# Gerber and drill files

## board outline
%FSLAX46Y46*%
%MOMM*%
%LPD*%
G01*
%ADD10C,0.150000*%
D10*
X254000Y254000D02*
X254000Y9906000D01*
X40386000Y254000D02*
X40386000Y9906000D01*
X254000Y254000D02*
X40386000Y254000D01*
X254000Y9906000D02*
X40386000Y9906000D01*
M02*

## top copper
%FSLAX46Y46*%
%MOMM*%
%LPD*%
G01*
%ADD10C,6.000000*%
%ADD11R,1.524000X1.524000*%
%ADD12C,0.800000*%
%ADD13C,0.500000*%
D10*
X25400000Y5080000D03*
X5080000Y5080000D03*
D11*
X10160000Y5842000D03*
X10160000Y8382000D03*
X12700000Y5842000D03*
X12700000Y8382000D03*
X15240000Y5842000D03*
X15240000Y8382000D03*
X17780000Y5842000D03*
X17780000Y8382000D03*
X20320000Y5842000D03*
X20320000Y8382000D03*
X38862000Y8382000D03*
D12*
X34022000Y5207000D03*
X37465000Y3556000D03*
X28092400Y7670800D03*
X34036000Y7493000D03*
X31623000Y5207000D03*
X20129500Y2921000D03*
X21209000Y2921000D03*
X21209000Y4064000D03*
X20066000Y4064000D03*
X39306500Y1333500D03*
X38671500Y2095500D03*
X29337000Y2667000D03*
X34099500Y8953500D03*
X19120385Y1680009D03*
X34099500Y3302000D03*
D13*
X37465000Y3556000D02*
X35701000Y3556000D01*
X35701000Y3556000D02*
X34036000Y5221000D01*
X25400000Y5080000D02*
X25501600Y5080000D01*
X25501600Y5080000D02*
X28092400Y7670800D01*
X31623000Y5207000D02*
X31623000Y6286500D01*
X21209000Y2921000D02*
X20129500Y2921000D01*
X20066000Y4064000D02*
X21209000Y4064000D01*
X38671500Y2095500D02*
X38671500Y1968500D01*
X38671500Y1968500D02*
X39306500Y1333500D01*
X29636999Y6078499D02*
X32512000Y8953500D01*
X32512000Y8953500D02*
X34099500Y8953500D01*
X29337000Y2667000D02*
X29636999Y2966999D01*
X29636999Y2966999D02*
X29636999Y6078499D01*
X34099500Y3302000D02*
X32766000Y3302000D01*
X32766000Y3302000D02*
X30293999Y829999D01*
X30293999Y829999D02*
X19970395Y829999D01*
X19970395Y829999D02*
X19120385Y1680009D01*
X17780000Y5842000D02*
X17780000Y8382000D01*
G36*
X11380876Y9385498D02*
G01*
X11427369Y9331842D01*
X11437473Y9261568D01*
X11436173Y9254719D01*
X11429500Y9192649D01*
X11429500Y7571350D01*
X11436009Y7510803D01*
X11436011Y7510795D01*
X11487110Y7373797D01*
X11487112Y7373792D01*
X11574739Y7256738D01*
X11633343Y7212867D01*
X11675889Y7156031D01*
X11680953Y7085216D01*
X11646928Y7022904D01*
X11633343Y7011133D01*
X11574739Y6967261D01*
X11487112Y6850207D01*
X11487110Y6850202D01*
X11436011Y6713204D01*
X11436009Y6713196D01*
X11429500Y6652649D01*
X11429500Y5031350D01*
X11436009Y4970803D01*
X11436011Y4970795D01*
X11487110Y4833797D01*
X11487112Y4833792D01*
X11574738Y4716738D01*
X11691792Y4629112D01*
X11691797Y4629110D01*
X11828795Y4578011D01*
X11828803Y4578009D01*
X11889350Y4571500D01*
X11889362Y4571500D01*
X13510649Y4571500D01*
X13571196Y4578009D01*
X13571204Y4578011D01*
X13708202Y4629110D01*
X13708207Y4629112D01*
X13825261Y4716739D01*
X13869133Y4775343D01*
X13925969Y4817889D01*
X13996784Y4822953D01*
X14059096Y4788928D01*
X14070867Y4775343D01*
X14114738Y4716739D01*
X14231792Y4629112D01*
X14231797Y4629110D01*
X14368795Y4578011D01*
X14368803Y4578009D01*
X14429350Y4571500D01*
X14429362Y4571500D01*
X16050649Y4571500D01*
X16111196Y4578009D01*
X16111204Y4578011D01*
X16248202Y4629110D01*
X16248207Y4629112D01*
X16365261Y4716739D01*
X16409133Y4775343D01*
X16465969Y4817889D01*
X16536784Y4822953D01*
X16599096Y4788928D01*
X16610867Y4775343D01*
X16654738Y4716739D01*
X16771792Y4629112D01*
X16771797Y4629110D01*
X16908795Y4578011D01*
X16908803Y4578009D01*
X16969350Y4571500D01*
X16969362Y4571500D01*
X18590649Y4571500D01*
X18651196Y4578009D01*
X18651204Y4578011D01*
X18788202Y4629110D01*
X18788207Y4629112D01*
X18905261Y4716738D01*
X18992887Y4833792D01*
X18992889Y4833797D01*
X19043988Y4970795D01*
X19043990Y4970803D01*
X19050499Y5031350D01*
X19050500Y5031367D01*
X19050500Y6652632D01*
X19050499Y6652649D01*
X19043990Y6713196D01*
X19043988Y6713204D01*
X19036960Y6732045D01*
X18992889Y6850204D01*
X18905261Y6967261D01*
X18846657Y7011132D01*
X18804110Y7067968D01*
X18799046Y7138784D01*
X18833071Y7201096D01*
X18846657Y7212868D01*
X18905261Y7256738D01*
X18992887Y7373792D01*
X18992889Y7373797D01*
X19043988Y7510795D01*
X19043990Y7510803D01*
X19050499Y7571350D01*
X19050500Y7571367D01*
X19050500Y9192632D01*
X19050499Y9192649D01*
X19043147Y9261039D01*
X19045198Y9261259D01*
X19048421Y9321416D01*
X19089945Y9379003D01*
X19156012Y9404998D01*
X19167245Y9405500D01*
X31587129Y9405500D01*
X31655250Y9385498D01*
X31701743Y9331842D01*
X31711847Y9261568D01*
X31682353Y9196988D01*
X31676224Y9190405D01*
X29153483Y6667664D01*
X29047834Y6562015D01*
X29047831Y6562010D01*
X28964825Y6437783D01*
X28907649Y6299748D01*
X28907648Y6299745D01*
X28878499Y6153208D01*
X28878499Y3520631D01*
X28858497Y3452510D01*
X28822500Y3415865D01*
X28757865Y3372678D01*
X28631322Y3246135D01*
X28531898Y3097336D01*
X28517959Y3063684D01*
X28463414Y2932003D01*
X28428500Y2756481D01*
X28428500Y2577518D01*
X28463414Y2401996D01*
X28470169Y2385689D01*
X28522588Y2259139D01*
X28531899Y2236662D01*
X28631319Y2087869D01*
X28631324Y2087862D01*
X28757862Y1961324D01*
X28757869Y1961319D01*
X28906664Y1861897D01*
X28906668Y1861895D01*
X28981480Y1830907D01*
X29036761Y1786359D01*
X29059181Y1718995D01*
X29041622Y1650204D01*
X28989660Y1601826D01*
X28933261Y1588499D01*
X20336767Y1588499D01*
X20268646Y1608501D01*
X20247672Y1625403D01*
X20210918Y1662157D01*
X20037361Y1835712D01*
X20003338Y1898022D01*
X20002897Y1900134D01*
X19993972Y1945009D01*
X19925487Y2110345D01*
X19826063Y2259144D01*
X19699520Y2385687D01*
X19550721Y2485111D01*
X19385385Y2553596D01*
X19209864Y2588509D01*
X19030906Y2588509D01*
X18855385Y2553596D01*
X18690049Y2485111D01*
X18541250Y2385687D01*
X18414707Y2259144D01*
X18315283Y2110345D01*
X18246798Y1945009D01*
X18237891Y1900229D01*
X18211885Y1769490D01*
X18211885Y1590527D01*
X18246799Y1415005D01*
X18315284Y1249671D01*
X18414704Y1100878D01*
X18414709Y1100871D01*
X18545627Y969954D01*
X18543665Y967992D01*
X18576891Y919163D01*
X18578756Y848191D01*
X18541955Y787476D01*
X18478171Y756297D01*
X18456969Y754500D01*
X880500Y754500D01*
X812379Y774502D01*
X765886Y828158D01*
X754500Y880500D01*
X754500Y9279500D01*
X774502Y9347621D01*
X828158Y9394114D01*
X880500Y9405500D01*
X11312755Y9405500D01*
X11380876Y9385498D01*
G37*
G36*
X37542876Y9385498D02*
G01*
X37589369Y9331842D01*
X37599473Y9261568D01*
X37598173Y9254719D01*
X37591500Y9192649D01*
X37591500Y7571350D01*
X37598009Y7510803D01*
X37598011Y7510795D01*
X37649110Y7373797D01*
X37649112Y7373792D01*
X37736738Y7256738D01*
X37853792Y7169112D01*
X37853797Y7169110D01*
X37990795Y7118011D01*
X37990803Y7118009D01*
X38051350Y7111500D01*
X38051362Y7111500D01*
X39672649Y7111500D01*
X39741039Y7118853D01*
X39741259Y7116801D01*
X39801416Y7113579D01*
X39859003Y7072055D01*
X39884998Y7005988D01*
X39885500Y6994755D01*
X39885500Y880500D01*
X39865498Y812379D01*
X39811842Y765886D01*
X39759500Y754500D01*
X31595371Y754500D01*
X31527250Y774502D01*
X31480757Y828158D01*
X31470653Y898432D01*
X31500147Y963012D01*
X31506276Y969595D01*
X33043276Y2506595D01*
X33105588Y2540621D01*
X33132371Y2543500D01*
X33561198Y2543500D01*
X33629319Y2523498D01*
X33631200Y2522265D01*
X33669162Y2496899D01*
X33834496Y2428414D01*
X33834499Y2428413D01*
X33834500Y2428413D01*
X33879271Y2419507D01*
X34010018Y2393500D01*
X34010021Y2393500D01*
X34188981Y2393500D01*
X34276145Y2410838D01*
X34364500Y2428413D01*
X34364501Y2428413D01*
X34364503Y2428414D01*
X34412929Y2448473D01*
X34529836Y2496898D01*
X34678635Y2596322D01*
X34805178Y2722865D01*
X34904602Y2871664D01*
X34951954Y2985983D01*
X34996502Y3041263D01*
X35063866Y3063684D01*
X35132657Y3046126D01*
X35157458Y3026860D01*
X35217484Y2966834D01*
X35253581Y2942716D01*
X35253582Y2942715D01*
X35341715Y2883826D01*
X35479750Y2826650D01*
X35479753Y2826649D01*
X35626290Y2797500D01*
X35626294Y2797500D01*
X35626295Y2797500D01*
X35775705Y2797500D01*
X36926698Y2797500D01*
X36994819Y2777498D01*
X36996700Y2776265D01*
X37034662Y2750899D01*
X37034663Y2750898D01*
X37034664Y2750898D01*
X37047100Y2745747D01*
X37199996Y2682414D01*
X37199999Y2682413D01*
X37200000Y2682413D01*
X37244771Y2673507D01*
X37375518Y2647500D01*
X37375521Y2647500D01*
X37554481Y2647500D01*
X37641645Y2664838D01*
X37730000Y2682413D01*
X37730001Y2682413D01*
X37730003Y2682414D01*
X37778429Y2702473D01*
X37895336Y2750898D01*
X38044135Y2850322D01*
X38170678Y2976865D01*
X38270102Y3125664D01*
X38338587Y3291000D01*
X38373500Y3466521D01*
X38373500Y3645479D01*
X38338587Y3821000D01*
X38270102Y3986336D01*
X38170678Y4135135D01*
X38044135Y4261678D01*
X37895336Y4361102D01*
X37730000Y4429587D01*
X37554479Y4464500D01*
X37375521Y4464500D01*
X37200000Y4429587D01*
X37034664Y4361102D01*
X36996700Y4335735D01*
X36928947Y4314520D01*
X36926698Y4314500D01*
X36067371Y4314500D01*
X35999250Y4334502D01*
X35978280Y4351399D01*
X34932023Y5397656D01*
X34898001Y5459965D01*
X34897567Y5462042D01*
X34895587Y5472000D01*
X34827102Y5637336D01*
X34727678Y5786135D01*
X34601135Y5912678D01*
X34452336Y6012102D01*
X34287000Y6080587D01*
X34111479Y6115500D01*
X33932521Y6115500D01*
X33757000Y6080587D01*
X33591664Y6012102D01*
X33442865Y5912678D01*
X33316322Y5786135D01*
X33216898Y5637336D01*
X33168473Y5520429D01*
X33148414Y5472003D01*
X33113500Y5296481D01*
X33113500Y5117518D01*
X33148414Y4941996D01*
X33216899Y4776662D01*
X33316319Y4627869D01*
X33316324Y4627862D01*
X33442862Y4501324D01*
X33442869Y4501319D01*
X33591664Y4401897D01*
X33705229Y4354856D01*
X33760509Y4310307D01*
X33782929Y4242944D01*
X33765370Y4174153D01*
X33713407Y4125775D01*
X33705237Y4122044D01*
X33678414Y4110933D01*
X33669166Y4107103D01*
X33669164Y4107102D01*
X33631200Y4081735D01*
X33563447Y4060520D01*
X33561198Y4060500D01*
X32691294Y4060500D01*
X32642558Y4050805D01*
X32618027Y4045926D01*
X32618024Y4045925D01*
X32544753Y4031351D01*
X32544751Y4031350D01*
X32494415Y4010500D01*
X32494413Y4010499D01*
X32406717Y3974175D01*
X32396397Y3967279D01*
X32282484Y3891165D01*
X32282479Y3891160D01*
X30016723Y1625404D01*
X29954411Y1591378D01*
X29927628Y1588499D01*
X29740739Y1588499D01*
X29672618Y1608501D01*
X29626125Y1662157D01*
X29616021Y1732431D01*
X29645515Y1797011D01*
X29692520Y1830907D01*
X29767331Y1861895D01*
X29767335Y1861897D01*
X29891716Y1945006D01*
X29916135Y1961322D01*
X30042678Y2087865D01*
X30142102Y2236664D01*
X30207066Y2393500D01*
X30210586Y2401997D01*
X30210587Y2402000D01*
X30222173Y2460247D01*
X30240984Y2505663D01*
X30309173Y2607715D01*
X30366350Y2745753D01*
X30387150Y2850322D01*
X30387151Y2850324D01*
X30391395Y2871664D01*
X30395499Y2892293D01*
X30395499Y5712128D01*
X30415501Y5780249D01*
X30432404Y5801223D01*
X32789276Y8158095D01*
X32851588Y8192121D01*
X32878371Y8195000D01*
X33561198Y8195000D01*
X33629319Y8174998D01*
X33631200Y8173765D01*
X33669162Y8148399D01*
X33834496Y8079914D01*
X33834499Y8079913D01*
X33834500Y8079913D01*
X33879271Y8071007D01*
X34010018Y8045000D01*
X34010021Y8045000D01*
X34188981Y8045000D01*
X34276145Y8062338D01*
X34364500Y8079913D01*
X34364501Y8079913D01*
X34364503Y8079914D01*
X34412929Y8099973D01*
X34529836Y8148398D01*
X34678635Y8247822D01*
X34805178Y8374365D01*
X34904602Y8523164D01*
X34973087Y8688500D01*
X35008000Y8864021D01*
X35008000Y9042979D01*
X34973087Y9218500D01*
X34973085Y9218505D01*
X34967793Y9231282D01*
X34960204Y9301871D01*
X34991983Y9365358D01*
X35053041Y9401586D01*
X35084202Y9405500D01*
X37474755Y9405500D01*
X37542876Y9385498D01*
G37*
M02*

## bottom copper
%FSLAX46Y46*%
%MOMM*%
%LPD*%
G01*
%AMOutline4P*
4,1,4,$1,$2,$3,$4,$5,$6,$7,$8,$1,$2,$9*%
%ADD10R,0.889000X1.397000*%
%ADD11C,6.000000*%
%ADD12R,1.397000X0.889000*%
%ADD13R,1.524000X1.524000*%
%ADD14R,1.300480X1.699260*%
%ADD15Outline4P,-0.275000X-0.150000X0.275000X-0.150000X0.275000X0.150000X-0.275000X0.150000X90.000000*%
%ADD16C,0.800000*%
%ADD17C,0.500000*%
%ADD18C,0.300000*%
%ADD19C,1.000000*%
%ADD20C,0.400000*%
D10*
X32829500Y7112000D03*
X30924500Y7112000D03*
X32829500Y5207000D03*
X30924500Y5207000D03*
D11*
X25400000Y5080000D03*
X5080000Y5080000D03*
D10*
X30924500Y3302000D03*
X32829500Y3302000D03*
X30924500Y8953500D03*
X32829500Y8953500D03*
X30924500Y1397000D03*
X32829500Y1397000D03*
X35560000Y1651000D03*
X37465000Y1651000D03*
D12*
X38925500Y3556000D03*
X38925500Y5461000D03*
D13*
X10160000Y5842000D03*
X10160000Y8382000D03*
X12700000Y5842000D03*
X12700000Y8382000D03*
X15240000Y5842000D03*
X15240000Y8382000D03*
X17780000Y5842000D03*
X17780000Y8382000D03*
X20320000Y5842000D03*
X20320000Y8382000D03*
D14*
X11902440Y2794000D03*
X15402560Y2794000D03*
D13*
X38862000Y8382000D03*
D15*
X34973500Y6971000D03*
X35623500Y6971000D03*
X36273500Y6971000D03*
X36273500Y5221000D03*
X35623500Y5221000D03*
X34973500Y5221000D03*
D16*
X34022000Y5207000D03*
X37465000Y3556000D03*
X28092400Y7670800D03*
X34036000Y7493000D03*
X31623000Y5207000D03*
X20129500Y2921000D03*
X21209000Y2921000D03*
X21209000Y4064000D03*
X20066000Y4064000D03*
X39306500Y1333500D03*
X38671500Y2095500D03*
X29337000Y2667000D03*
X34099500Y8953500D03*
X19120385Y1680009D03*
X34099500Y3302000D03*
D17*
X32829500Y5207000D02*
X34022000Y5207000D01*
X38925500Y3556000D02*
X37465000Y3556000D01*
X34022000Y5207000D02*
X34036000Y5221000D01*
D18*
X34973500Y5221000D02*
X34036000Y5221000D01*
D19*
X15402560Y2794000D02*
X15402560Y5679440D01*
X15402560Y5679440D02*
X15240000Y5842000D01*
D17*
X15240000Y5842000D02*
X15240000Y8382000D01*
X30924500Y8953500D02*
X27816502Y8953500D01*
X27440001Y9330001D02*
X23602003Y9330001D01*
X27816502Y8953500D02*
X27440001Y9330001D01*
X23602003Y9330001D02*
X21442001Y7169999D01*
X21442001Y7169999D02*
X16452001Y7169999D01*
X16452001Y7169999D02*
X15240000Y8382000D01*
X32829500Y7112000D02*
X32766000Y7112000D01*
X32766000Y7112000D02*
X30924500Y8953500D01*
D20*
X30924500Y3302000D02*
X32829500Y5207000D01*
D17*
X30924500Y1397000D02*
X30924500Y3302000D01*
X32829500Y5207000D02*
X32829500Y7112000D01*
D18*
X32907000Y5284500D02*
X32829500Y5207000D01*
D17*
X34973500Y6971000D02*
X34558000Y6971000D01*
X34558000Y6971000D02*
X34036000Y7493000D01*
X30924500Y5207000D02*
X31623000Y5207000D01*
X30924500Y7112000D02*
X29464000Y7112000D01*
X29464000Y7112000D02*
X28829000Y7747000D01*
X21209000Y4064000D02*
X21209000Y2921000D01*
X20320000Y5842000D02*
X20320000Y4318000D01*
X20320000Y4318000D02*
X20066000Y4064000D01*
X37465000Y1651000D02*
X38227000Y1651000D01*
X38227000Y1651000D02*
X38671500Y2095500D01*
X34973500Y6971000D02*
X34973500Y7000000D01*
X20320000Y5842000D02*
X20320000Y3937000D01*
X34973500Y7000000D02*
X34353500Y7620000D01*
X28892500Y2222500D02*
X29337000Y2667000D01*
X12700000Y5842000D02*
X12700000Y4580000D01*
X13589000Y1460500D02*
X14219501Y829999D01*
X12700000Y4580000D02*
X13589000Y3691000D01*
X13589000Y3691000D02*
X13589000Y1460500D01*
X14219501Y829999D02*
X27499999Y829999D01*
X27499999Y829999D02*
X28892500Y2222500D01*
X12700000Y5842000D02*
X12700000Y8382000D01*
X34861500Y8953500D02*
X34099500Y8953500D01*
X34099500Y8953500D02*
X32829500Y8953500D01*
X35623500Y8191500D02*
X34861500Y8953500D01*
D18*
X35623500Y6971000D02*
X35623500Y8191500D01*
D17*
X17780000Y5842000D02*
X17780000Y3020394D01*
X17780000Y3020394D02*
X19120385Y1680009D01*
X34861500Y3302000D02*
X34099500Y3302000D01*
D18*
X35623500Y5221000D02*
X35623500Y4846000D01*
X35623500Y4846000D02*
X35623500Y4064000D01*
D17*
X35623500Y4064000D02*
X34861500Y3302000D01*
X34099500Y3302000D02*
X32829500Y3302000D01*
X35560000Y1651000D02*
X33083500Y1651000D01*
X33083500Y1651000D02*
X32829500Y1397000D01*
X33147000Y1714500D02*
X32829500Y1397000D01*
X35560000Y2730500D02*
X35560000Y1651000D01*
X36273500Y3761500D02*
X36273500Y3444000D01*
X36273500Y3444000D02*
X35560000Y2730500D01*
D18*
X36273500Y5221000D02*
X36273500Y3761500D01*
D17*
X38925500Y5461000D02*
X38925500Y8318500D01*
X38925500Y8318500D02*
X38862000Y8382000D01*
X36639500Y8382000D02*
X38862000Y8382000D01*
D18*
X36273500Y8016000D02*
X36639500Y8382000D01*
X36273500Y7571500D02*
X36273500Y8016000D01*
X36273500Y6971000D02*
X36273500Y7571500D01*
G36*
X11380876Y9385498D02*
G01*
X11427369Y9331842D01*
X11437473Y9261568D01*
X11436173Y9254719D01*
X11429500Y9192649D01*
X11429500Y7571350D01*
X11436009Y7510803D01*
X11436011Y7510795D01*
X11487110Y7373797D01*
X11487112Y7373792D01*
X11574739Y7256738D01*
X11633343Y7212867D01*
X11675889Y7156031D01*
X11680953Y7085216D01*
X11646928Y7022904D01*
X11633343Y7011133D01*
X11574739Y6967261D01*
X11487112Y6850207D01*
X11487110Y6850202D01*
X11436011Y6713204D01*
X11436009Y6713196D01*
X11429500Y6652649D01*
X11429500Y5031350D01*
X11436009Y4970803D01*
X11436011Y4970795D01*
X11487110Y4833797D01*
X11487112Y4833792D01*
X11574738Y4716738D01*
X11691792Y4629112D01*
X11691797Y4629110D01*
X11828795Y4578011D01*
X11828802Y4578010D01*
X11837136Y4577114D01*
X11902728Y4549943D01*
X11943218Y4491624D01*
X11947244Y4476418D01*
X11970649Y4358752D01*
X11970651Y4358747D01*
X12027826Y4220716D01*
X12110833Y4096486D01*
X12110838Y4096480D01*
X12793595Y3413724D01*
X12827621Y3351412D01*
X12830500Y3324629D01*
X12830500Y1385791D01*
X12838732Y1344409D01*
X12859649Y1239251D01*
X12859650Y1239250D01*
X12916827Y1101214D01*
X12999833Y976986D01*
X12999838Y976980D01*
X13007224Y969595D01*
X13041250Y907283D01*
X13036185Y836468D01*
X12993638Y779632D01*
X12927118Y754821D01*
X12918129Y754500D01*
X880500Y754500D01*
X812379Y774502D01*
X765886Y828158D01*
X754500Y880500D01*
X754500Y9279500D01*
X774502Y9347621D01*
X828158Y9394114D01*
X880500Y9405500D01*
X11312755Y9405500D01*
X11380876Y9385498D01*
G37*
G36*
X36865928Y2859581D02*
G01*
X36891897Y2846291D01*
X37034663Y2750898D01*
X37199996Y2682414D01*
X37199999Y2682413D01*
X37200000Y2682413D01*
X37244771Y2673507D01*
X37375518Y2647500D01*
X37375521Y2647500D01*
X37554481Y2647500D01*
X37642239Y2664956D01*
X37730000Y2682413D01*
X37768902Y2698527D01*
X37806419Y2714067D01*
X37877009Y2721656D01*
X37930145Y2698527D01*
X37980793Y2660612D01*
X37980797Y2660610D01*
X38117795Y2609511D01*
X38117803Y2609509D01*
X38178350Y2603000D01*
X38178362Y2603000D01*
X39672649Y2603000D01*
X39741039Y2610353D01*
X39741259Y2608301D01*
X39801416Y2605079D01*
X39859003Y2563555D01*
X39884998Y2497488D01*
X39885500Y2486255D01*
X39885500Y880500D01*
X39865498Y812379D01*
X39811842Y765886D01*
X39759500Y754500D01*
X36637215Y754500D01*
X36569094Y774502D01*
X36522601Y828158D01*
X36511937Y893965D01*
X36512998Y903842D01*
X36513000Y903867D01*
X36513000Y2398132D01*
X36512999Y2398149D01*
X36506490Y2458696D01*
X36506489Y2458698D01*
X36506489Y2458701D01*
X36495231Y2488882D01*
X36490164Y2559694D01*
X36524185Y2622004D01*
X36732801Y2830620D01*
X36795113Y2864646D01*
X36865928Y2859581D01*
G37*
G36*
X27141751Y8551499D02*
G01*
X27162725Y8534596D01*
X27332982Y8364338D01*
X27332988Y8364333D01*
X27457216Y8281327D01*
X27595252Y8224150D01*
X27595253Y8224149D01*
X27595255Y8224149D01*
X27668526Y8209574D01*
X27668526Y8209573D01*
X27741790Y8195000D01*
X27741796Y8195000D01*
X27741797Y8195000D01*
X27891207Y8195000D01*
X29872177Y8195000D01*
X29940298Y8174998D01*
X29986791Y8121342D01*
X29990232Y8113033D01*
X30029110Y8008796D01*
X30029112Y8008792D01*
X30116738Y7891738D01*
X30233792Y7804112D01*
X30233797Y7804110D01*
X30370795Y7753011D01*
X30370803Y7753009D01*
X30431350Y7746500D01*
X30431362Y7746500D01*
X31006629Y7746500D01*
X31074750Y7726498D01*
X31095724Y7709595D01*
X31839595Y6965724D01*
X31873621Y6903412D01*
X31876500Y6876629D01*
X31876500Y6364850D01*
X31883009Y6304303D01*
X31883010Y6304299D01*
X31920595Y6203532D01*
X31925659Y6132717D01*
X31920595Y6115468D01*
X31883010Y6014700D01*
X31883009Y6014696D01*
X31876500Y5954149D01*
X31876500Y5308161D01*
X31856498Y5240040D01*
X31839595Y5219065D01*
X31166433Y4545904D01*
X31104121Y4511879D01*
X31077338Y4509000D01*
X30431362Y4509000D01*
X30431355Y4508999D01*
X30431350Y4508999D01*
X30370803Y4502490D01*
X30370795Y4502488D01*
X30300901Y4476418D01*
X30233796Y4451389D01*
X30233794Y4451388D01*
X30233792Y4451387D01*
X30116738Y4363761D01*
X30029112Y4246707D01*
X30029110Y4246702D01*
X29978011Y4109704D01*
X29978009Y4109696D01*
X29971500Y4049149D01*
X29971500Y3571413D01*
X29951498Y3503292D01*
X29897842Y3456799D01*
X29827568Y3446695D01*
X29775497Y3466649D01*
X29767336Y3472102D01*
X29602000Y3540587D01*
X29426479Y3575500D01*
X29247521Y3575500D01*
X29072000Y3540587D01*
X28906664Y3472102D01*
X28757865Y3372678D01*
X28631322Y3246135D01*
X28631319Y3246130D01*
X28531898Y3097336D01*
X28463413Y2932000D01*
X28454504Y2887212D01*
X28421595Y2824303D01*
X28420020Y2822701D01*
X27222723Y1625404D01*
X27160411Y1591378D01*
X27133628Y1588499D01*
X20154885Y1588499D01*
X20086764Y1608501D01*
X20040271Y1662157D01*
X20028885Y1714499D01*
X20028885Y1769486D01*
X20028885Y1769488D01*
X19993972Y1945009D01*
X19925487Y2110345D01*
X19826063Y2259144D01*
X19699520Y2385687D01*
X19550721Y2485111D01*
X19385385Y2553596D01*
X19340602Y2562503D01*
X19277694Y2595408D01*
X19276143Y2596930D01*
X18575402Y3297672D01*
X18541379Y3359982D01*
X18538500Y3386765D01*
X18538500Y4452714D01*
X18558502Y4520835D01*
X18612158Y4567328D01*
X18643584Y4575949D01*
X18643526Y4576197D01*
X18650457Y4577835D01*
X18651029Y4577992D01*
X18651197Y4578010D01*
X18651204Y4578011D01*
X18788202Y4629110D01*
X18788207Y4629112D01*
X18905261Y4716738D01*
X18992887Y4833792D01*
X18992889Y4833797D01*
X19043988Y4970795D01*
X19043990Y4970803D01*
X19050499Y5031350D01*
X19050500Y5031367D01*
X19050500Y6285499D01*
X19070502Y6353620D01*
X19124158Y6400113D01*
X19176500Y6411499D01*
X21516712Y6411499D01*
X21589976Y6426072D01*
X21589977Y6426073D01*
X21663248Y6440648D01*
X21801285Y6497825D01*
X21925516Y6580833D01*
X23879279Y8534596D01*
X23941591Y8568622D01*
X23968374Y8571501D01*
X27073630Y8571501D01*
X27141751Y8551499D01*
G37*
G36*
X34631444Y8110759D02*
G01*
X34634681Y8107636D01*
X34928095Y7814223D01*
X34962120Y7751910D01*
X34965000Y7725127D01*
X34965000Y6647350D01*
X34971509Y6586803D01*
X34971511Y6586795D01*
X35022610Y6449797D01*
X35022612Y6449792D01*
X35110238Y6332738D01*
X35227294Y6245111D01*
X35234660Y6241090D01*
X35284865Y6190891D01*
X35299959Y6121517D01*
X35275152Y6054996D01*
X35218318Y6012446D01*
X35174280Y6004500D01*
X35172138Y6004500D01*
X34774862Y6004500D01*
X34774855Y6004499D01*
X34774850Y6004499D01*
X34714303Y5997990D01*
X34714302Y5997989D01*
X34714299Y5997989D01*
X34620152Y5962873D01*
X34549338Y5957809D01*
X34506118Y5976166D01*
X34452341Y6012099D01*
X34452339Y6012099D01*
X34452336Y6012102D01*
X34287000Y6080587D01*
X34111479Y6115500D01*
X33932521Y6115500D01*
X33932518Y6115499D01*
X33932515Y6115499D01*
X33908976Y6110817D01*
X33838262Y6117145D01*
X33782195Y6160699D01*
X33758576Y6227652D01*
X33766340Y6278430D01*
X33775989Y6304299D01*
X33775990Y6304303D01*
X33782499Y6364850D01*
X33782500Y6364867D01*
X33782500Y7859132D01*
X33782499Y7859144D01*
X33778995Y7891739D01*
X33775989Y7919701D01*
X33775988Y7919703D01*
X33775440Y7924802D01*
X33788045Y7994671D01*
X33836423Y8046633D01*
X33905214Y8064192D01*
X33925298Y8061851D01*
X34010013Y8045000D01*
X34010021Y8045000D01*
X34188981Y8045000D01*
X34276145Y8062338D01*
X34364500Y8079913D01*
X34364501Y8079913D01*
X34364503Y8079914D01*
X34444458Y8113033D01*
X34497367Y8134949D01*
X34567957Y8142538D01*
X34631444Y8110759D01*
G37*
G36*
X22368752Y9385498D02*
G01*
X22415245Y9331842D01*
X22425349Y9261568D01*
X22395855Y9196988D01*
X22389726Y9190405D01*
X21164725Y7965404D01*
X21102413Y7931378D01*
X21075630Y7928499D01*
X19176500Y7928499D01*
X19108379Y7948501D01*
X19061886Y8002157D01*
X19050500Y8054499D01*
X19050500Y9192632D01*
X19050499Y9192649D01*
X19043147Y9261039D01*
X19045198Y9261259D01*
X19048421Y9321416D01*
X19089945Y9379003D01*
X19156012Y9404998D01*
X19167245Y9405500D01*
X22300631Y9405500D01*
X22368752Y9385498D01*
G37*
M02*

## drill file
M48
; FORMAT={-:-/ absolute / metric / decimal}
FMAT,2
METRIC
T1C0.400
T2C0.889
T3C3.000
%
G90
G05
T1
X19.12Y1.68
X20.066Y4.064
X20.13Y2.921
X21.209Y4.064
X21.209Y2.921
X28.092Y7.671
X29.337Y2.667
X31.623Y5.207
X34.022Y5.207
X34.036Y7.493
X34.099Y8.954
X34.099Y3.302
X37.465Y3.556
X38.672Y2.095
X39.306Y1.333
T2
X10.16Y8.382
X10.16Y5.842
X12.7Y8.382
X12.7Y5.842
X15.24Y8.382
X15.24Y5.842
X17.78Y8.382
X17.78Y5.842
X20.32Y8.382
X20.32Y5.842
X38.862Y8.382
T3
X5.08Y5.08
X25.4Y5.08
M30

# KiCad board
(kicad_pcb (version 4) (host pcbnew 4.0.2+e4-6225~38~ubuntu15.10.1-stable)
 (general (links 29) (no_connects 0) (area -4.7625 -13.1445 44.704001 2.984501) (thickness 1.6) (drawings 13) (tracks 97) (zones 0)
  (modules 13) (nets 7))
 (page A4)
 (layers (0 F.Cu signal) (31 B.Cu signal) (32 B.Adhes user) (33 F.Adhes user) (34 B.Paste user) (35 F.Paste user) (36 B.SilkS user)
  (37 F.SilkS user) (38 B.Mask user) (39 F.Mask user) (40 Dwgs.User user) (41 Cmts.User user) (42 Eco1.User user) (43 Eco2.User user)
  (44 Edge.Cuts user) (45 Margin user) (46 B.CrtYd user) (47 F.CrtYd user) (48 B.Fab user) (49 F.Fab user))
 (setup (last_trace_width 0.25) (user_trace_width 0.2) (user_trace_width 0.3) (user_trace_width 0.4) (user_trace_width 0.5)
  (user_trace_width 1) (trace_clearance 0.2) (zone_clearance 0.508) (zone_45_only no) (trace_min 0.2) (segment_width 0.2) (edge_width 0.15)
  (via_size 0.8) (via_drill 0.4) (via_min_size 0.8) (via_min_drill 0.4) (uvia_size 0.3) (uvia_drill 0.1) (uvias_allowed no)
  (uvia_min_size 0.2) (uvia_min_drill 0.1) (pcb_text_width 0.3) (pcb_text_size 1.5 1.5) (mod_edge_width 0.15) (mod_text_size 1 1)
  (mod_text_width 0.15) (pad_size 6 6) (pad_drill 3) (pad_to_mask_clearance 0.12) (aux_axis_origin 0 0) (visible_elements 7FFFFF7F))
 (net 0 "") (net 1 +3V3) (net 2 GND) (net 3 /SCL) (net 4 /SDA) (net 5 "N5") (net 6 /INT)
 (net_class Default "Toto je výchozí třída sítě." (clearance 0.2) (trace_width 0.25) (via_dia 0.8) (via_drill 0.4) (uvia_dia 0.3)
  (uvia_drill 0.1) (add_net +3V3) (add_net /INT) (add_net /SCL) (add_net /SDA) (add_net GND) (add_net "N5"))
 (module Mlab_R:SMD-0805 (layer B.Cu) (at 31.877 -7.112 180)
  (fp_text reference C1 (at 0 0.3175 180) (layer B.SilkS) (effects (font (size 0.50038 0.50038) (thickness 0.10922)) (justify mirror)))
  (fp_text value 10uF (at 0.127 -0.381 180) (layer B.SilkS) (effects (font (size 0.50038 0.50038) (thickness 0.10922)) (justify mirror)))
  (pad 1 smd rect (at -0.9525 0 180) (size 0.889 1.397) (layers B.Cu B.Paste B.Mask) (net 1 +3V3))
  (pad 2 smd rect (at 0.9525 0 180) (size 0.889 1.397) (layers B.Cu B.Paste B.Mask) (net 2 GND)))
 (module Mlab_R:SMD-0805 (layer B.Cu) (at 31.877 -5.207 180)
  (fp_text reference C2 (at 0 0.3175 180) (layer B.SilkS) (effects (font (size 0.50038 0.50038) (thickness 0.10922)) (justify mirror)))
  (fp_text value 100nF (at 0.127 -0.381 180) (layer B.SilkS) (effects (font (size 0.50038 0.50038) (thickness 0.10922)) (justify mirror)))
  (pad 1 smd rect (at -0.9525 0 180) (size 0.889 1.397) (layers B.Cu B.Paste B.Mask) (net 1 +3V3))
  (pad 2 smd rect (at 0.9525 0 180) (size 0.889 1.397) (layers B.Cu B.Paste B.Mask) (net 2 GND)))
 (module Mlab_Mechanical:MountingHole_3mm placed (layer F.Cu) (at 25.4 -5.08)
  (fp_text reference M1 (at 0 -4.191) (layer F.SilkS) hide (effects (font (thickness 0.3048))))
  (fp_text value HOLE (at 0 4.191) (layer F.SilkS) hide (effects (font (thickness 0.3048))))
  (pad 1 thru_hole circle (at 0 0) (size 6 6) (drill 3) (layers *.Cu *.Adhes *.Mask) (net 2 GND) (clearance 1) (zone_connect 2)))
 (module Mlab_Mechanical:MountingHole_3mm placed (layer F.Cu) (at 5.08 -5.08)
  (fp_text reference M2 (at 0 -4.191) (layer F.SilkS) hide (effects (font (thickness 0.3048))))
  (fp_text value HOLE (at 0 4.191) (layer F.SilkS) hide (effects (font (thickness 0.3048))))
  (pad 1 thru_hole circle (at 0 0) (size 6 6) (drill 3) (layers *.Cu *.Adhes *.Mask) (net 2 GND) (clearance 1) (zone_connect 2)))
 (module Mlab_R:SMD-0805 (layer B.Cu) (at 31.877 -3.302)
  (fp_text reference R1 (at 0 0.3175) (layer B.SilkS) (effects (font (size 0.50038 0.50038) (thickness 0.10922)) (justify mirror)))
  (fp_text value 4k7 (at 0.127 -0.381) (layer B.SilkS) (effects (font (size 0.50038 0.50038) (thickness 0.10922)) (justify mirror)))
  (pad 1 smd rect (at -0.9525 0) (size 0.889 1.397) (layers B.Cu B.Paste B.Mask) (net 1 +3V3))
  (pad 2 smd rect (at 0.9525 0) (size 0.889 1.397) (layers B.Cu B.Paste B.Mask) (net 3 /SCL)))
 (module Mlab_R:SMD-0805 (layer B.Cu) (at 31.877 -8.9535)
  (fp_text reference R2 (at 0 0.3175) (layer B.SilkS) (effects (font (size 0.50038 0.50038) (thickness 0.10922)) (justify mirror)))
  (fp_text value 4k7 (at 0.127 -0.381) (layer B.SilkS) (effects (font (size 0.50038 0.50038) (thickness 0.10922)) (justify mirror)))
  (pad 1 smd rect (at -0.9525 0) (size 0.889 1.397) (layers B.Cu B.Paste B.Mask) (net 1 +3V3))
  (pad 2 smd rect (at 0.9525 0) (size 0.889 1.397) (layers B.Cu B.Paste B.Mask) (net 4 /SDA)))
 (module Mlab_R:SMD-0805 (layer B.Cu) (at 31.877 -1.397)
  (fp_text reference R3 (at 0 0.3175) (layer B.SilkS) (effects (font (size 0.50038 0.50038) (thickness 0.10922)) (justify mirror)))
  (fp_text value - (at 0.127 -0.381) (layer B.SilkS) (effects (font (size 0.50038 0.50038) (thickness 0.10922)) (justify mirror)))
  (pad 1 smd rect (at -0.9525 0) (size 0.889 1.397) (layers B.Cu B.Paste B.Mask) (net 1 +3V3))
  (pad 2 smd rect (at 0.9525 0) (size 0.889 1.397) (layers B.Cu B.Paste B.Mask) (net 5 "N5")))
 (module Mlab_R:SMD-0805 (layer B.Cu) (at 36.5125 -1.651)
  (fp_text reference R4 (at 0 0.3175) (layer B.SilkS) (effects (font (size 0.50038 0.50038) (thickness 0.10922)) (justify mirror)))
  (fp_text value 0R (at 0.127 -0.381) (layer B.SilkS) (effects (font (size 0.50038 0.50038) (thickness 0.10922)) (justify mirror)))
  (pad 1 smd rect (at -0.9525 0) (size 0.889 1.397) (layers B.Cu B.Paste B.Mask) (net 5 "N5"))
  (pad 2 smd rect (at 0.9525 0) (size 0.889 1.397) (layers B.Cu B.Paste B.Mask) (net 2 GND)))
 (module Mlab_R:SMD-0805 (layer B.Cu) (at 38.9255 -4.5085 90)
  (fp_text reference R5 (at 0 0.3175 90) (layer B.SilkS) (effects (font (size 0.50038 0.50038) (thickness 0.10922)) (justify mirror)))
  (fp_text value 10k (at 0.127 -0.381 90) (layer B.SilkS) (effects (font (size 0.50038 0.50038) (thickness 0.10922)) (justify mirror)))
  (pad 1 smd rect (at -0.9525 0 90) (size 0.889 1.397) (layers B.Cu B.Paste B.Mask) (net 1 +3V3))
  (pad 2 smd rect (at 0.9525 0 90) (size 0.889 1.397) (layers B.Cu B.Paste B.Mask) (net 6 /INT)))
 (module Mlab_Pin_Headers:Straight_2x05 (layer F.Cu) (at 15.24 -7.112 90)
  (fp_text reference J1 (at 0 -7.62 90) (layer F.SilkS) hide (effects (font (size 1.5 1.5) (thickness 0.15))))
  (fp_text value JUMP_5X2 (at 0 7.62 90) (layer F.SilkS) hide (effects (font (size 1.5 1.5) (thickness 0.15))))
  (pad 1 thru_hole rect (at -1.27 -5.08 90) (size 1.524 1.524) (drill 0.889) (layers *.Cu *.Mask F.SilkS) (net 2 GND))
  (pad 2 thru_hole rect (at 1.27 -5.08 90) (size 1.524 1.524) (drill 0.889) (layers *.Cu *.Mask F.SilkS) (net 2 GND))
  (pad 3 thru_hole rect (at -1.27 -2.54 90) (size 1.524 1.524) (drill 0.889) (layers *.Cu *.Mask F.SilkS) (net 4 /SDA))
  (pad 4 thru_hole rect (at 1.27 -2.54 90) (size 1.524 1.524) (drill 0.889) (layers *.Cu *.Mask F.SilkS) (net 4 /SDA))
  (pad 5 thru_hole rect (at -1.27 0 90) (size 1.524 1.524) (drill 0.889) (layers *.Cu *.Mask F.SilkS) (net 1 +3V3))
  (pad 6 thru_hole rect (at 1.27 0 90) (size 1.524 1.524) (drill 0.889) (layers *.Cu *.Mask F.SilkS) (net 1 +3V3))
  (pad 7 thru_hole rect (at -1.27 2.54 90) (size 1.524 1.524) (drill 0.889) (layers *.Cu *.Mask F.SilkS) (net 3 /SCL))
  (pad 8 thru_hole rect (at 1.27 2.54 90) (size 1.524 1.524) (drill 0.889) (layers *.Cu *.Mask F.SilkS) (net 3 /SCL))
  (pad 9 thru_hole rect (at -1.27 5.08 90) (size 1.524 1.524) (drill 0.889) (layers *.Cu *.Mask F.SilkS) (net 2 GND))
  (pad 10 thru_hole rect (at 1.27 5.08 90) (size 1.524 1.524) (drill 0.889) (layers *.Cu *.Mask F.SilkS) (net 2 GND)))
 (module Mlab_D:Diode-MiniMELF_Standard (layer B.Cu) (at 13.6525 -2.794)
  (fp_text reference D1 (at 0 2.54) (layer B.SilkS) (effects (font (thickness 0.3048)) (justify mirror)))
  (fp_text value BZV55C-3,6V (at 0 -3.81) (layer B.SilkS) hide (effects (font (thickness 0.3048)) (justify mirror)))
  (pad 1 smd rect (at -1.75006 0) (size 1.30048 1.69926) (layers B.Cu B.Paste B.Mask) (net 2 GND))
  (pad 2 smd rect (at 1.75006 0) (size 1.30048 1.69926) (layers B.Cu B.Paste B.Mask) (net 1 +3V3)))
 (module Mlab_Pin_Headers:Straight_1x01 (layer F.Cu) (at 38.862 -8.382)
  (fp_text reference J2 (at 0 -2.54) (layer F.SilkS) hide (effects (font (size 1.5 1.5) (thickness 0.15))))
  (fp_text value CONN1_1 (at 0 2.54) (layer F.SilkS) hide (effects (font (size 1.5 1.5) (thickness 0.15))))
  (pad 1 thru_hole rect (at 0 0) (size 1.524 1.524) (drill 0.889) (layers *.Cu *.Mask F.SilkS) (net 6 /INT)))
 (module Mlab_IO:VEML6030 (layer B.Cu) (at 35.6235 -6.096 90)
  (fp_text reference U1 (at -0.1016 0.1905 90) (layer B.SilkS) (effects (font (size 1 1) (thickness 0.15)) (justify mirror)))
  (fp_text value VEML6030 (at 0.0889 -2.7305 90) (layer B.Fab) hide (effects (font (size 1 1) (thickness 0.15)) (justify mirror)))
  (pad 1 smd trapezoid (at 0.875 -0.65 90) (size 0.55 0.3) (layers B.Cu B.Paste B.Mask) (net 2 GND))
  (pad 2 smd trapezoid (at 0.875 0 90) (size 0.55 0.3) (layers B.Cu B.Paste B.Mask) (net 4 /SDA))
  (pad 3 smd trapezoid (at 0.875 0.65 90) (size 0.55 0.3) (layers B.Cu B.Paste B.Mask) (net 6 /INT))
  (pad 4 smd trapezoid (at -0.875 0.65 90) (size 0.55 0.3) (layers B.Cu B.Paste B.Mask) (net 5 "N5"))
  (pad 5 smd trapezoid (at -0.875 0 90) (size 0.55 0.3) (layers B.Cu B.Paste B.Mask) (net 3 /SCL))
  (pad 6 smd trapezoid (at -0.875 -0.65 90) (size 0.55 0.3) (layers B.Cu B.Paste B.Mask) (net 1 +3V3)))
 (gr_line (start 0.254 -0.254) (end 0.254 -9.906) (angle 90) (layer Edge.Cuts) (width 0.15))
 (gr_line (start 40.386 -0.254) (end 40.386 -9.906) (angle 90) (layer Edge.Cuts) (width 0.15))
 (gr_line (start 0.254 -0.254) (end 40.386 -0.254) (angle 90) (layer Edge.Cuts) (width 0.15))
 (gr_line (start 0.254 -9.906) (end 40.386 -9.906) (angle 90) (layer Edge.Cuts) (width 0.15))
 (segment (start 32.8295 -5.207) (end 34.022 -5.207) (width 0.5) (layer B.Cu) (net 1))
 (via (at 34.022 -5.207) (size 0.8) (drill 0.4) (layers F.Cu B.Cu) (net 1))
 (segment (start 38.9255 -3.556) (end 37.465 -3.556) (width 0.5) (layer B.Cu) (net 1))
 (via (at 37.465 -3.556) (size 0.8) (drill 0.4) (layers F.Cu B.Cu) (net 1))
 (segment (start 34.022 -5.207) (end 34.036 -5.221) (width 0.5) (layer B.Cu) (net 1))
 (segment (start 34.9735 -5.221) (end 34.036 -5.221) (width 0.3) (layer B.Cu) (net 1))
 (segment (start 37.465 -3.556) (end 35.701 -3.556) (width 0.5) (layer F.Cu) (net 1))
 (segment (start 35.701 -3.556) (end 34.036 -5.221) (width 0.5) (layer F.Cu) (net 1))
 (segment (start 15.40256 -2.794) (end 15.40256 -5.67944) (width 1) (layer B.Cu) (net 1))
 (segment (start 15.40256 -5.67944) (end 15.24 -5.842) (width 1) (layer B.Cu) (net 1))
 (segment (start 15.24 -5.842) (end 15.24 -8.382) (width 0.5) (layer B.Cu) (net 1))
 (segment (start 30.9245 -8.9535) (end 27.816502 -8.9535) (width 0.5) (layer B.Cu) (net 1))
 (segment (start 27.440001 -9.330001) (end 23.602003 -9.330001) (width 0.5) (layer B.Cu) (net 1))
 (segment (start 27.816502 -8.9535) (end 27.440001 -9.330001) (width 0.5) (layer B.Cu) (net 1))
 (segment (start 23.602003 -9.330001) (end 21.442001 -7.169999) (width 0.5) (layer B.Cu) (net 1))
 (segment (start 21.442001 -7.169999) (end 16.452001 -7.169999) (width 0.5) (layer B.Cu) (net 1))
 (segment (start 16.452001 -7.169999) (end 15.24 -8.382) (width 0.5) (layer B.Cu) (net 1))
 (segment (start 32.8295 -7.112) (end 32.766 -7.112) (width 0.5) (layer B.Cu) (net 1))
 (segment (start 32.766 -7.112) (end 30.9245 -8.9535) (width 0.5) (layer B.Cu) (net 1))
 (segment (start 30.9245 -3.302) (end 32.8295 -5.207) (width 0.4) (layer B.Cu) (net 1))
 (segment (start 30.9245 -1.397) (end 30.9245 -3.302) (width 0.5) (layer B.Cu) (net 1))
 (segment (start 32.8295 -5.207) (end 32.8295 -7.112) (width 0.5) (layer B.Cu) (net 1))
 (segment (start 32.907 -5.2845) (end 32.8295 -5.207) (width 0.3) (layer B.Cu) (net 1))
 (segment (start 25.4 -5.08) (end 25.5016 -5.08) (width 0.5) (layer F.Cu) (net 2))
 (segment (start 25.5016 -5.08) (end 28.0924 -7.6708) (width 0.5) (layer F.Cu) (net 2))
 (via (at 28.0924 -7.6708) (size 0.8) (drill 0.4) (layers F.Cu B.Cu) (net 2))
 (segment (start 34.9735 -6.971) (end 34.558 -6.971) (width 0.5) (layer B.Cu) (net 2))
 (segment (start 34.558 -6.971) (end 34.036 -7.493) (width 0.5) (layer B.Cu) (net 2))
 (via (at 34.036 -7.493) (size 0.8) (drill 0.4) (layers F.Cu B.Cu) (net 2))
 (segment (start 31.623 -5.207) (end 31.623 -6.2865) (width 0.5) (layer F.Cu) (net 2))
 (segment (start 30.9245 -5.207) (end 31.623 -5.207) (width 0.5) (layer B.Cu) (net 2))
 (via (at 31.623 -5.207) (size 0.8) (drill 0.4) (layers F.Cu B.Cu) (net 2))
 (segment (start 30.9245 -7.112) (end 29.464 -7.112) (width 0.5) (layer B.Cu) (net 2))
 (segment (start 29.464 -7.112) (end 28.829 -7.747) (width 0.5) (layer B.Cu) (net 2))
 (segment (start 21.209 -2.921) (end 20.1295 -2.921) (width 0.5) (layer F.Cu) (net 2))
 (via (at 20.1295 -2.921) (size 0.8) (drill 0.4) (layers F.Cu B.Cu) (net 2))
 (segment (start 21.209 -4.064) (end 21.209 -2.921) (width 0.5) (layer B.Cu) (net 2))
 (via (at 21.209 -2.921) (size 0.8) (drill 0.4) (layers F.Cu B.Cu) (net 2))
 (segment (start 20.066 -4.064) (end 21.209 -4.064) (width 0.5) (layer F.Cu) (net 2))
 (via (at 21.209 -4.064) (size 0.8) (drill 0.4) (layers F.Cu B.Cu) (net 2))
 (segment (start 20.32 -5.842) (end 20.32 -4.318) (width 0.5) (layer B.Cu) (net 2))
 (segment (start 20.32 -4.318) (end 20.066 -4.064) (width 0.5) (layer B.Cu) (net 2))
 (via (at 20.066 -4.064) (size 0.8) (drill 0.4) (layers F.Cu B.Cu) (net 2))
 (segment (start 38.6715 -2.0955) (end 38.6715 -1.9685) (width 0.5) (layer F.Cu) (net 2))
 (segment (start 38.6715 -1.9685) (end 39.3065 -1.3335) (width 0.5) (layer F.Cu) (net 2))
 (via (at 39.3065 -1.3335) (size 0.8) (drill 0.4) (layers F.Cu B.Cu) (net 2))
 (segment (start 37.465 -1.651) (end 38.227 -1.651) (width 0.5) (layer B.Cu) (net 2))
 (segment (start 38.227 -1.651) (end 38.6715 -2.0955) (width 0.5) (layer B.Cu) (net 2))
 (via (at 38.6715 -2.0955) (size 0.8) (drill 0.4) (layers F.Cu B.Cu) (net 2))
 (segment (start 34.9735 -6.971) (end 34.9735 -7) (width 0.5) (layer B.Cu) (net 2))
 (segment (start 20.32 -5.842) (end 20.32 -3.937) (width 0.5) (layer B.Cu) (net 2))
 (segment (start 34.9735 -7) (end 34.3535 -7.62) (width 0.5) (layer B.Cu) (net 2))
 (segment (start 28.8925 -2.2225) (end 29.337 -2.667) (width 0.5) (layer B.Cu) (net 4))
 (via (at 29.337 -2.667) (size 0.8) (drill 0.4) (layers F.Cu B.Cu) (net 4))
 (segment (start 12.7 -5.842) (end 12.7 -4.58) (width 0.5) (layer B.Cu) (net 4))
 (segment (start 13.589 -1.4605) (end 14.219501 -0.829999) (width 0.5) (layer B.Cu) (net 4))
 (segment (start 12.7 -4.58) (end 13.589 -3.691) (width 0.5) (layer B.Cu) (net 4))
 (segment (start 13.589 -3.691) (end 13.589 -1.4605) (width 0.5) (layer B.Cu) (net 4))
 (segment (start 14.219501 -0.829999) (end 27.499999 -0.829999) (width 0.5) (layer B.Cu) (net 4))
 (segment (start 27.499999 -0.829999) (end 28.8925 -2.2225) (width 0.5) (layer B.Cu) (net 4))
 (via (at 34.0995 -8.9535) (size 0.8) (drill 0.4) (layers F.Cu B.Cu) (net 4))
 (segment (start 12.7 -5.842) (end 12.7 -8.382) (width 0.5) (layer B.Cu) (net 4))
 (segment (start 34.8615 -8.9535) (end 34.0995 -8.9535) (width 0.5) (layer B.Cu) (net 4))
 (segment (start 34.0995 -8.9535) (end 32.8295 -8.9535) (width 0.5) (layer B.Cu) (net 4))
 (segment (start 29.636999 -6.078499) (end 32.512 -8.9535) (width 0.5) (layer F.Cu) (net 4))
 (segment (start 32.512 -8.9535) (end 34.0995 -8.9535) (width 0.5) (layer F.Cu) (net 4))
 (segment (start 29.337 -2.667) (end 29.636999 -2.966999) (width 0.5) (layer F.Cu) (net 4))
 (segment (start 29.636999 -2.966999) (end 29.636999 -6.078499) (width 0.5) (layer F.Cu) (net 4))
 (segment (start 35.6235 -8.1915) (end 34.8615 -8.9535) (width 0.5) (layer B.Cu) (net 4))
 (segment (start 35.6235 -6.971) (end 35.6235 -8.1915) (width 0.3) (layer B.Cu) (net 4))
 (segment (start 34.0995 -3.302) (end 32.766 -3.302) (width 0.5) (layer F.Cu) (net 3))
 (segment (start 32.766 -3.302) (end 30.293999 -0.829999) (width 0.5) (layer F.Cu) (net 3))
 (segment (start 30.293999 -0.829999) (end 19.970395 -0.829999) (width 0.5) (layer F.Cu) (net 3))
 (segment (start 19.970395 -0.829999) (end 19.120385 -1.680009) (width 0.5) (layer F.Cu) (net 3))
 (segment (start 17.78 -5.842) (end 17.78 -3.020394) (width 0.5) (layer B.Cu) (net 3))
 (segment (start 17.78 -3.020394) (end 19.120385 -1.680009) (width 0.5) (layer B.Cu) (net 3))
 (via (at 19.120385 -1.680009) (size 0.8) (drill 0.4) (layers F.Cu B.Cu) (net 3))
 (via (at 34.0995 -3.302) (size 0.8) (drill 0.4) (layers F.Cu B.Cu) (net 3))
 (segment (start 34.8615 -3.302) (end 34.0995 -3.302) (width 0.5) (layer B.Cu) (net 3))
 (segment (start 35.6235 -5.221) (end 35.6235 -4.846) (width 0.3) (layer B.Cu) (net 3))
 (segment (start 35.6235 -4.846) (end 35.6235 -4.064) (width 0.3) (layer B.Cu) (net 3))
 (segment (start 35.6235 -4.064) (end 34.8615 -3.302) (width 0.5) (layer B.Cu) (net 3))
 (segment (start 17.78 -5.842) (end 17.78 -8.382) (width 0.5) (layer F.Cu) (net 3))
 (segment (start 34.0995 -3.302) (end 32.8295 -3.302) (width 0.5) (layer B.Cu) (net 3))
 (segment (start 35.56 -1.651) (end 33.0835 -1.651) (width 0.5) (layer B.Cu) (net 5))
 (segment (start 33.0835 -1.651) (end 32.8295 -1.397) (width 0.5) (layer B.Cu) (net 5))
 (segment (start 33.147 -1.7145) (end 32.8295 -1.397) (width 0.5) (layer B.Cu) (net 5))
 (segment (start 35.56 -2.7305) (end 35.56 -1.651) (width 0.5) (layer B.Cu) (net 5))
 (segment (start 36.2735 -3.7615) (end 36.2735 -3.444) (width 0.5) (layer B.Cu) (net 5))
 (segment (start 36.2735 -3.444) (end 35.56 -2.7305) (width 0.5) (layer B.Cu) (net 5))
 (segment (start 36.2735 -5.221) (end 36.2735 -3.7615) (width 0.3) (layer B.Cu) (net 5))
 (segment (start 38.9255 -5.461) (end 38.9255 -8.3185) (width 0.5) (layer B.Cu) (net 6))
 (segment (start 38.9255 -8.3185) (end 38.862 -8.382) (width 0.5) (layer B.Cu) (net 6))
 (segment (start 36.6395 -8.382) (end 38.862 -8.382) (width 0.5) (layer B.Cu) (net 6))
 (segment (start 36.2735 -8.016) (end 36.6395 -8.382) (width 0.3) (layer B.Cu) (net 6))
 (segment (start 36.2735 -7.5715) (end 36.2735 -8.016) (width 0.3) (layer B.Cu) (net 6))
 (segment (start 36.2735 -6.971) (end 36.2735 -7.5715) (width 0.3) (layer B.Cu) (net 6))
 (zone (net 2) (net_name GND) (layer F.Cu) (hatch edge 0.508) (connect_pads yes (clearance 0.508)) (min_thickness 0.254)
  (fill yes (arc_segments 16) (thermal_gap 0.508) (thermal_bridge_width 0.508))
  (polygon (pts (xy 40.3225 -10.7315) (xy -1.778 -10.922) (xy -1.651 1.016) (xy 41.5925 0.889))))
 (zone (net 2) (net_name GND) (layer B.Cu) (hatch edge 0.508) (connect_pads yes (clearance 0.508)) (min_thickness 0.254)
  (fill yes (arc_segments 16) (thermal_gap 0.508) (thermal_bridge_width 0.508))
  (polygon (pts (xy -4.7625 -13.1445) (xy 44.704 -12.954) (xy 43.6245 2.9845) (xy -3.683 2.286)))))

